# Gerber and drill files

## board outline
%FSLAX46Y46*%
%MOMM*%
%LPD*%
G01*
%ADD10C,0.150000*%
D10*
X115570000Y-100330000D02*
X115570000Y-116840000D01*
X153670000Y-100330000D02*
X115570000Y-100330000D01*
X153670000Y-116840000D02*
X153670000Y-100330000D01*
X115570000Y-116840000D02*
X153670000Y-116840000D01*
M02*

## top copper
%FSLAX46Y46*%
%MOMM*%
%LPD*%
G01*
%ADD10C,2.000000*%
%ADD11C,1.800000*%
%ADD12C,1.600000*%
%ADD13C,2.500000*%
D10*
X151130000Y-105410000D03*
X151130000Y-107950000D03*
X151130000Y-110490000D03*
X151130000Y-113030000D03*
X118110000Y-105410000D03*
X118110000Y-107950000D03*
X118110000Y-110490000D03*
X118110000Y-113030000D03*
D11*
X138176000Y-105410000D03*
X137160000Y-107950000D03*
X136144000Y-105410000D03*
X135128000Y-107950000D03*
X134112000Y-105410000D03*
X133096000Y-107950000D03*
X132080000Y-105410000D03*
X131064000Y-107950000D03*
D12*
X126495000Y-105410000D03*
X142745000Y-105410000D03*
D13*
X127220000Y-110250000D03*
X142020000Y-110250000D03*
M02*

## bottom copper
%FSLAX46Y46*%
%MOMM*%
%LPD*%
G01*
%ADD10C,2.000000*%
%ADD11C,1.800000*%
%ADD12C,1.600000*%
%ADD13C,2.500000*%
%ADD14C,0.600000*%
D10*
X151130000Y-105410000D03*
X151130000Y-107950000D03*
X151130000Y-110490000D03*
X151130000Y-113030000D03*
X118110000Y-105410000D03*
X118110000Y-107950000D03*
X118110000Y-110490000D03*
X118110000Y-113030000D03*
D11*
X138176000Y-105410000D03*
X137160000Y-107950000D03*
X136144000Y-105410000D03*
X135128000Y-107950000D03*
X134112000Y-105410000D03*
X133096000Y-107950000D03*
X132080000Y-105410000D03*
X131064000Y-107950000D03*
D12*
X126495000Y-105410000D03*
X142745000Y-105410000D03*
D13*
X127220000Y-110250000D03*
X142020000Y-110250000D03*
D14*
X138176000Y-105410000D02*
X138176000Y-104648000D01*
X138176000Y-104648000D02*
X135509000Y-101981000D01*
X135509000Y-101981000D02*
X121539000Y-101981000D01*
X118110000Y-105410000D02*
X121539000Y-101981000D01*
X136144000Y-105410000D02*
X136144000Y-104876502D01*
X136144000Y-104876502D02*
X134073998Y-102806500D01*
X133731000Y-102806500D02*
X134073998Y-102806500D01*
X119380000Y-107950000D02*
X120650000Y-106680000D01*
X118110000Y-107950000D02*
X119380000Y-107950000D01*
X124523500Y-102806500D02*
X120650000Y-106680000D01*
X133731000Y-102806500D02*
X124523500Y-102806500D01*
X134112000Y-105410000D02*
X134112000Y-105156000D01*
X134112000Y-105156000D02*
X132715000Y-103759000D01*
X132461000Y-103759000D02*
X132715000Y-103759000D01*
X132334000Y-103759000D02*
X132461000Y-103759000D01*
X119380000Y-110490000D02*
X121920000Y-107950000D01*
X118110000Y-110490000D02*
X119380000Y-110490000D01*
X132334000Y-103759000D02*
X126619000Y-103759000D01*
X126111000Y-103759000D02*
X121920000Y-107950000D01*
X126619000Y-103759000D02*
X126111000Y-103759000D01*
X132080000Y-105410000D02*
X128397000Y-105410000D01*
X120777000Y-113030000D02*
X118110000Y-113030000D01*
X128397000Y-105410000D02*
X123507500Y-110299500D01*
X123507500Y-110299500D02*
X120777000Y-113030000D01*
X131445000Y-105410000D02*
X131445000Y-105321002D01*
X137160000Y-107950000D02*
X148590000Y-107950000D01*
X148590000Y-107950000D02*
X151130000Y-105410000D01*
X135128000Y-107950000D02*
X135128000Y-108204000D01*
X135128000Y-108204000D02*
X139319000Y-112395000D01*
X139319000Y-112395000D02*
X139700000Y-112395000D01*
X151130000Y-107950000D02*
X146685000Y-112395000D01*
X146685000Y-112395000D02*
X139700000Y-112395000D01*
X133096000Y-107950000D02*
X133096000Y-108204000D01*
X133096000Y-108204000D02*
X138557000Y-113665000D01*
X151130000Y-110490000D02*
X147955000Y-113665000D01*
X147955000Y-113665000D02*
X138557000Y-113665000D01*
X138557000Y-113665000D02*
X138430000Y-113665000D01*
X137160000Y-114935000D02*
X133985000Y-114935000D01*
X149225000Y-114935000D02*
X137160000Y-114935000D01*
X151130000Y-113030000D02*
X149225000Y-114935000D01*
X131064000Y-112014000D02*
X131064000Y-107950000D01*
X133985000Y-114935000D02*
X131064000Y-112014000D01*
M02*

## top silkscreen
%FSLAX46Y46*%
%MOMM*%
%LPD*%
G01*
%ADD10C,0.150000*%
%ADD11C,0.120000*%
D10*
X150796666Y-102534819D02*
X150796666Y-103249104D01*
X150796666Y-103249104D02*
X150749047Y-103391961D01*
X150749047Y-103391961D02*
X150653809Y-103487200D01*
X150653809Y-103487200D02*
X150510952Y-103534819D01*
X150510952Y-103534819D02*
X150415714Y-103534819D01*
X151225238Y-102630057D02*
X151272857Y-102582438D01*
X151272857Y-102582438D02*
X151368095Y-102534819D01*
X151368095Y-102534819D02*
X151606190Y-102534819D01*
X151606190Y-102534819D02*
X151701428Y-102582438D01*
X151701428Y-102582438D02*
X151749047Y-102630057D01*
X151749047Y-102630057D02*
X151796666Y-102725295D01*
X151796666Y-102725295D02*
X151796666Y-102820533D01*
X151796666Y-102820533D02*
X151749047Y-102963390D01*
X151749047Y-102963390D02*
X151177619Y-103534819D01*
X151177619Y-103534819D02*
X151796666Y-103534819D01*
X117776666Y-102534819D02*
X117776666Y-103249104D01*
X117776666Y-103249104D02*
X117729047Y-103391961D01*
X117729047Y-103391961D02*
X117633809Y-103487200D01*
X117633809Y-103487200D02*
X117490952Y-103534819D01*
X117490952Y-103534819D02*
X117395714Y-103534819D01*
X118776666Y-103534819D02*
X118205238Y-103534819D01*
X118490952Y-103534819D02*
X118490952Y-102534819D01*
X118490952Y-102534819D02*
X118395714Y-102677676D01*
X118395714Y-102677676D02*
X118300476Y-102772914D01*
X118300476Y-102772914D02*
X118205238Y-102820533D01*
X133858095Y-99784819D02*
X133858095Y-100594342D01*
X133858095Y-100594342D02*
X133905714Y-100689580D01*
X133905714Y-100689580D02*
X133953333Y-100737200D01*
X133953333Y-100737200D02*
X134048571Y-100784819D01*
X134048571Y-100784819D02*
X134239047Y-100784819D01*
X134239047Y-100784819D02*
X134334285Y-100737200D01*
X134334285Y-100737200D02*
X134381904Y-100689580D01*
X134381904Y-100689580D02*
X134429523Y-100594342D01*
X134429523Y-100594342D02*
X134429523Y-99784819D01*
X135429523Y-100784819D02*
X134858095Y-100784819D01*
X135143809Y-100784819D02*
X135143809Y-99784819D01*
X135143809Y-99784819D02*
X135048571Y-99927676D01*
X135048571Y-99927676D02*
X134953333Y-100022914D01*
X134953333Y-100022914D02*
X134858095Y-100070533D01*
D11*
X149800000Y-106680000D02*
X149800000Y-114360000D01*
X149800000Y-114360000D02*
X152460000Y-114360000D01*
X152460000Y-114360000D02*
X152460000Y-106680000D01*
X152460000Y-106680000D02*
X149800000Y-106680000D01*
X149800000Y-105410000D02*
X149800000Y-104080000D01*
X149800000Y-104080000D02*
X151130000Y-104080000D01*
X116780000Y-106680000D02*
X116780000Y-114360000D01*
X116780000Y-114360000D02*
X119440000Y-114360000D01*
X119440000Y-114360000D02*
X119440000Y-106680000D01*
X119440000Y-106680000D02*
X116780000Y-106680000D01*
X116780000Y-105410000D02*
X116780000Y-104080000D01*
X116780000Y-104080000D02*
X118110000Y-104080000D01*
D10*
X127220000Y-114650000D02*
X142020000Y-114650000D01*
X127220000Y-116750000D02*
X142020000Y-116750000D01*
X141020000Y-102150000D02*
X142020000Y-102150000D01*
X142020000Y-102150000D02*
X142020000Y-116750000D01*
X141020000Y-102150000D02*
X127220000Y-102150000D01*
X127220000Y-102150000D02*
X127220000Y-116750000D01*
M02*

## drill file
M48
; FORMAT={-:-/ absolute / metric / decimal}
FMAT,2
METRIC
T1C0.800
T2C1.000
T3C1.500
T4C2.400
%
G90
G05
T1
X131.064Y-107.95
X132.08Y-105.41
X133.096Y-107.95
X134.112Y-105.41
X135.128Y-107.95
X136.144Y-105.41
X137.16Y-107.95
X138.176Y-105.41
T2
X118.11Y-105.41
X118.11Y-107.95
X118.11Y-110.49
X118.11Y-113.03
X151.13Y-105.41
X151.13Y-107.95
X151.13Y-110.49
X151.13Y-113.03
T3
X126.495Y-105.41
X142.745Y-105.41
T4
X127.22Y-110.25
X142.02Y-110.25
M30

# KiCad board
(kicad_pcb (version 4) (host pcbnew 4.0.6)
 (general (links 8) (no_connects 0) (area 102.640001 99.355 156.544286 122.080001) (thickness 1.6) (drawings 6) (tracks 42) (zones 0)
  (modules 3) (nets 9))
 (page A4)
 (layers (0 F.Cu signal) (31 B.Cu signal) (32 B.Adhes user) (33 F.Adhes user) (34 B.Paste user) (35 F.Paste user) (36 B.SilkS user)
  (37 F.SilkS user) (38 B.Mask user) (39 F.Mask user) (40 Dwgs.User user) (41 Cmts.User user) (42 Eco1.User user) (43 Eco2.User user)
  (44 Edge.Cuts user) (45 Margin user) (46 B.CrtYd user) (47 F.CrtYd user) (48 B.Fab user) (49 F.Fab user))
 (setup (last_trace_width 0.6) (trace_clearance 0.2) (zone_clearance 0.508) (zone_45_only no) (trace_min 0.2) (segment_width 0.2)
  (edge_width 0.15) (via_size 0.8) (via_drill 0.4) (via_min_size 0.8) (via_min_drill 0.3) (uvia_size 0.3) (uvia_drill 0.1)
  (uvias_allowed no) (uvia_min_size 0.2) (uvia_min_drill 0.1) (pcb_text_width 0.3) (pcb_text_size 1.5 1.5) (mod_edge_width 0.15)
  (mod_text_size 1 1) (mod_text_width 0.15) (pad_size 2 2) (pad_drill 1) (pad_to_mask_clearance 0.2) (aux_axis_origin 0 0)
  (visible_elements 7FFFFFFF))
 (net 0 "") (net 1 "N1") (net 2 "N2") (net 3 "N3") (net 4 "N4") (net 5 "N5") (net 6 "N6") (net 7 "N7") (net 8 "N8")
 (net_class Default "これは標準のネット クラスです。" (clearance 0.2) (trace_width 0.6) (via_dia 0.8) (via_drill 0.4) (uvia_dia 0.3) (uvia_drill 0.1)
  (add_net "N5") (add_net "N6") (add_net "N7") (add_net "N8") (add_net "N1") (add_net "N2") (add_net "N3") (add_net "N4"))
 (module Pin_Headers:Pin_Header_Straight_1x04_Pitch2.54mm (layer F.Cu) (at 151.13 105.41)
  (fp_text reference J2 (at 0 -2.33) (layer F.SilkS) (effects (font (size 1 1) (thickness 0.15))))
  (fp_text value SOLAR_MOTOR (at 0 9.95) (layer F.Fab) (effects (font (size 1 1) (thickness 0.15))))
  (fp_line (start -1.33 1.27) (end -1.33 8.95) (layer F.SilkS) (width 0.12))
  (fp_line (start -1.33 8.95) (end 1.33 8.95) (layer F.SilkS) (width 0.12))
  (fp_line (start 1.33 8.95) (end 1.33 1.27) (layer F.SilkS) (width 0.12))
  (fp_line (start 1.33 1.27) (end -1.33 1.27) (layer F.SilkS) (width 0.12))
  (fp_line (start -1.33 0) (end -1.33 -1.33) (layer F.SilkS) (width 0.12))
  (fp_line (start -1.33 -1.33) (end 0 -1.33) (layer F.SilkS) (width 0.12))
  (pad 1 thru_hole circle (at 0 0) (size 2 2) (drill 1) (layers *.Cu *.Mask) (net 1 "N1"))
  (pad 2 thru_hole circle (at 0 2.54) (size 2 2) (drill 1) (layers *.Cu *.Mask) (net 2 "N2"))
  (pad 3 thru_hole circle (at 0 5.08) (size 2 2) (drill 1) (layers *.Cu *.Mask) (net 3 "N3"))
  (pad 4 thru_hole circle (at 0 7.62) (size 2 2) (drill 1) (layers *.Cu *.Mask) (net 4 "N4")))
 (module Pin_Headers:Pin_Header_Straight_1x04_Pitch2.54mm (layer F.Cu) (at 118.11 105.41)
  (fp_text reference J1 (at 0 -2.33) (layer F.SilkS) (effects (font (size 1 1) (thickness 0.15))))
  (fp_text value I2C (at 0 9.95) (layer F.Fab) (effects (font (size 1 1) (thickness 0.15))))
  (fp_line (start -1.33 1.27) (end -1.33 8.95) (layer F.SilkS) (width 0.12))
  (fp_line (start -1.33 8.95) (end 1.33 8.95) (layer F.SilkS) (width 0.12))
  (fp_line (start 1.33 8.95) (end 1.33 1.27) (layer F.SilkS) (width 0.12))
  (fp_line (start 1.33 1.27) (end -1.33 1.27) (layer F.SilkS) (width 0.12))
  (fp_line (start -1.33 0) (end -1.33 -1.33) (layer F.SilkS) (width 0.12))
  (fp_line (start -1.33 -1.33) (end 0 -1.33) (layer F.SilkS) (width 0.12))
  (pad 1 thru_hole circle (at 0 0) (size 2 2) (drill 1) (layers *.Cu *.Mask) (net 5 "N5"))
  (pad 2 thru_hole circle (at 0 2.54) (size 2 2) (drill 1) (layers *.Cu *.Mask) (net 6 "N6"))
  (pad 3 thru_hole circle (at 0 5.08) (size 2 2) (drill 1) (layers *.Cu *.Mask) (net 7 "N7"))
  (pad 4 thru_hole circle (at 0 7.62) (size 2 2) (drill 1) (layers *.Cu *.Mask) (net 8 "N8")))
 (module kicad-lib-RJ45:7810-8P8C (layer F.Cu) (at 134.62 107.95)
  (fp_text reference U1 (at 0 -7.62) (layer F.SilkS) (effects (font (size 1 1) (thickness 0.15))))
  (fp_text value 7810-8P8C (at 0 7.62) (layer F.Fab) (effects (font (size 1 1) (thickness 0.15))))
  (fp_line (start -7.4 6.7) (end 7.4 6.7) (layer F.SilkS) (width 0.15))
  (fp_line (start -7.4 8.8) (end 7.4 8.8) (layer F.SilkS) (width 0.15))
  (fp_line (start 6.4 -5.8) (end 7.4 -5.8) (layer F.SilkS) (width 0.15))
  (fp_line (start 7.4 -5.8) (end 7.4 8.8) (layer F.SilkS) (width 0.15))
  (fp_line (start 6.4 -5.8) (end -7.4 -5.8) (layer F.SilkS) (width 0.15))
  (fp_line (start -7.4 -5.8) (end -7.4 8.8) (layer F.SilkS) (width 0.15))
  (pad 1 thru_hole circle (at 3.556 -2.54) (size 1.8 1.8) (drill 0.8) (layers *.Cu *.Mask) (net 5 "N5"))
  (pad 2 thru_hole circle (at 2.54 0) (size 1.8 1.8) (drill 0.8) (layers *.Cu *.Mask) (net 1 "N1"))
  (pad 3 thru_hole circle (at 1.524 -2.54) (size 1.8 1.8) (drill 0.8) (layers *.Cu *.Mask) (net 6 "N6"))
  (pad 4 thru_hole circle (at 0.508 0) (size 1.8 1.8) (drill 0.8) (layers *.Cu *.Mask) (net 2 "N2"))
  (pad 5 thru_hole circle (at -0.508 -2.54) (size 1.8 1.8) (drill 0.8) (layers *.Cu *.Mask) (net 7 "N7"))
  (pad 6 thru_hole circle (at -1.524 0) (size 1.8 1.8) (drill 0.8) (layers *.Cu *.Mask) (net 3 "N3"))
  (pad 7 thru_hole circle (at -2.54 -2.54) (size 1.8 1.8) (drill 0.8) (layers *.Cu *.Mask) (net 8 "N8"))
  (pad 8 thru_hole circle (at -3.556 0) (size 1.8 1.8) (drill 0.8) (layers *.Cu *.Mask) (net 4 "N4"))
  (pad "" np_thru_hole circle (at -8.125 -2.54) (size 1.6 1.6) (drill 1.5) (layers *.Cu *.Mask))
  (pad "" np_thru_hole circle (at 8.125 -2.54) (size 1.6 1.6) (drill 1.5) (layers *.Cu *.Mask))
  (pad "" np_thru_hole circle (at -7.4 2.3) (size 2.5 2.5) (drill 2.4) (layers *.Cu *.Mask))
  (pad "" np_thru_hole circle (at 7.4 2.3) (size 2.5 2.5) (drill 2.4) (layers *.Cu *.Mask)))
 (gr_line (start 115.57 100.33) (end 115.57 116.84) (angle 90) (layer Edge.Cuts) (width 0.15))
 (gr_line (start 153.67 100.33) (end 115.57 100.33) (angle 90) (layer Edge.Cuts) (width 0.15))
 (gr_line (start 153.67 116.84) (end 153.67 100.33) (angle 90) (layer Edge.Cuts) (width 0.15))
 (gr_line (start 115.57 116.84) (end 153.67 116.84) (angle 90) (layer Edge.Cuts) (width 0.15))
 (segment (start 138.176 105.41) (end 138.176 104.648) (width 0.6) (layer B.Cu) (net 5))
 (segment (start 138.176 104.648) (end 135.509 101.981) (width 0.6) (layer B.Cu) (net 5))
 (segment (start 135.509 101.981) (end 121.539 101.981) (width 0.6) (layer B.Cu) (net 5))
 (segment (start 118.11 105.41) (end 121.539 101.981) (width 0.6) (layer B.Cu) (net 5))
 (segment (start 136.144 105.41) (end 136.144 104.876502) (width 0.6) (layer B.Cu) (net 6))
 (segment (start 136.144 104.876502) (end 134.073998 102.8065) (width 0.6) (layer B.Cu) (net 6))
 (segment (start 133.731 102.8065) (end 134.073998 102.8065) (width 0.6) (layer B.Cu) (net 6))
 (segment (start 119.38 107.95) (end 120.65 106.68) (width 0.6) (layer B.Cu) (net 6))
 (segment (start 118.11 107.95) (end 119.38 107.95) (width 0.6) (layer B.Cu) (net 6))
 (segment (start 124.5235 102.8065) (end 120.65 106.68) (width 0.6) (layer B.Cu) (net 6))
 (segment (start 133.731 102.8065) (end 124.5235 102.8065) (width 0.6) (layer B.Cu) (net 6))
 (segment (start 134.112 105.41) (end 134.112 105.156) (width 0.6) (layer B.Cu) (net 7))
 (segment (start 134.112 105.156) (end 132.715 103.759) (width 0.6) (layer B.Cu) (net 7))
 (segment (start 132.461 103.759) (end 132.715 103.759) (width 0.6) (layer B.Cu) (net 7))
 (segment (start 132.334 103.759) (end 132.461 103.759) (width 0.6) (layer B.Cu) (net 7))
 (segment (start 119.38 110.49) (end 121.92 107.95) (width 0.6) (layer B.Cu) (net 7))
 (segment (start 118.11 110.49) (end 119.38 110.49) (width 0.6) (layer B.Cu) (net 7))
 (segment (start 132.334 103.759) (end 126.619 103.759) (width 0.6) (layer B.Cu) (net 7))
 (segment (start 126.111 103.759) (end 121.92 107.95) (width 0.6) (layer B.Cu) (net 7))
 (segment (start 126.619 103.759) (end 126.111 103.759) (width 0.6) (layer B.Cu) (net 7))
 (segment (start 132.08 105.41) (end 128.397 105.41) (width 0.6) (layer B.Cu) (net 8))
 (segment (start 120.777 113.03) (end 118.11 113.03) (width 0.6) (layer B.Cu) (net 8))
 (segment (start 128.397 105.41) (end 123.5075 110.2995) (width 0.6) (layer B.Cu) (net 8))
 (segment (start 123.5075 110.2995) (end 120.777 113.03) (width 0.6) (layer B.Cu) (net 8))
 (segment (start 131.445 105.41) (end 131.445 105.321002) (width 0.6) (layer B.Cu) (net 8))
 (segment (start 137.16 107.95) (end 148.59 107.95) (width 0.6) (layer B.Cu) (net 1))
 (segment (start 148.59 107.95) (end 151.13 105.41) (width 0.6) (layer B.Cu) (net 1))
 (segment (start 135.128 107.95) (end 135.128 108.204) (width 0.6) (layer B.Cu) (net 2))
 (segment (start 135.128 108.204) (end 139.319 112.395) (width 0.6) (layer B.Cu) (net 2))
 (segment (start 139.319 112.395) (end 139.7 112.395) (width 0.6) (layer B.Cu) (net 2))
 (segment (start 151.13 107.95) (end 146.685 112.395) (width 0.6) (layer B.Cu) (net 2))
 (segment (start 146.685 112.395) (end 139.7 112.395) (width 0.6) (layer B.Cu) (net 2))
 (segment (start 133.096 107.95) (end 133.096 108.204) (width 0.6) (layer B.Cu) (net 3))
 (segment (start 133.096 108.204) (end 138.557 113.665) (width 0.6) (layer B.Cu) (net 3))
 (segment (start 151.13 110.49) (end 147.955 113.665) (width 0.6) (layer B.Cu) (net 3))
 (segment (start 147.955 113.665) (end 138.557 113.665) (width 0.6) (layer B.Cu) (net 3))
 (segment (start 138.557 113.665) (end 138.43 113.665) (width 0.6) (layer B.Cu) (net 3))
 (segment (start 137.16 114.935) (end 133.985 114.935) (width 0.6) (layer B.Cu) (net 4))
 (segment (start 149.225 114.935) (end 137.16 114.935) (width 0.6) (layer B.Cu) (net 4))
 (segment (start 151.13 113.03) (end 149.225 114.935) (width 0.6) (layer B.Cu) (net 4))
 (segment (start 131.064 112.014) (end 131.064 107.95) (width 0.6) (layer B.Cu) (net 4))
 (segment (start 133.985 114.935) (end 131.064 112.014) (width 0.6) (layer B.Cu) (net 4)))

